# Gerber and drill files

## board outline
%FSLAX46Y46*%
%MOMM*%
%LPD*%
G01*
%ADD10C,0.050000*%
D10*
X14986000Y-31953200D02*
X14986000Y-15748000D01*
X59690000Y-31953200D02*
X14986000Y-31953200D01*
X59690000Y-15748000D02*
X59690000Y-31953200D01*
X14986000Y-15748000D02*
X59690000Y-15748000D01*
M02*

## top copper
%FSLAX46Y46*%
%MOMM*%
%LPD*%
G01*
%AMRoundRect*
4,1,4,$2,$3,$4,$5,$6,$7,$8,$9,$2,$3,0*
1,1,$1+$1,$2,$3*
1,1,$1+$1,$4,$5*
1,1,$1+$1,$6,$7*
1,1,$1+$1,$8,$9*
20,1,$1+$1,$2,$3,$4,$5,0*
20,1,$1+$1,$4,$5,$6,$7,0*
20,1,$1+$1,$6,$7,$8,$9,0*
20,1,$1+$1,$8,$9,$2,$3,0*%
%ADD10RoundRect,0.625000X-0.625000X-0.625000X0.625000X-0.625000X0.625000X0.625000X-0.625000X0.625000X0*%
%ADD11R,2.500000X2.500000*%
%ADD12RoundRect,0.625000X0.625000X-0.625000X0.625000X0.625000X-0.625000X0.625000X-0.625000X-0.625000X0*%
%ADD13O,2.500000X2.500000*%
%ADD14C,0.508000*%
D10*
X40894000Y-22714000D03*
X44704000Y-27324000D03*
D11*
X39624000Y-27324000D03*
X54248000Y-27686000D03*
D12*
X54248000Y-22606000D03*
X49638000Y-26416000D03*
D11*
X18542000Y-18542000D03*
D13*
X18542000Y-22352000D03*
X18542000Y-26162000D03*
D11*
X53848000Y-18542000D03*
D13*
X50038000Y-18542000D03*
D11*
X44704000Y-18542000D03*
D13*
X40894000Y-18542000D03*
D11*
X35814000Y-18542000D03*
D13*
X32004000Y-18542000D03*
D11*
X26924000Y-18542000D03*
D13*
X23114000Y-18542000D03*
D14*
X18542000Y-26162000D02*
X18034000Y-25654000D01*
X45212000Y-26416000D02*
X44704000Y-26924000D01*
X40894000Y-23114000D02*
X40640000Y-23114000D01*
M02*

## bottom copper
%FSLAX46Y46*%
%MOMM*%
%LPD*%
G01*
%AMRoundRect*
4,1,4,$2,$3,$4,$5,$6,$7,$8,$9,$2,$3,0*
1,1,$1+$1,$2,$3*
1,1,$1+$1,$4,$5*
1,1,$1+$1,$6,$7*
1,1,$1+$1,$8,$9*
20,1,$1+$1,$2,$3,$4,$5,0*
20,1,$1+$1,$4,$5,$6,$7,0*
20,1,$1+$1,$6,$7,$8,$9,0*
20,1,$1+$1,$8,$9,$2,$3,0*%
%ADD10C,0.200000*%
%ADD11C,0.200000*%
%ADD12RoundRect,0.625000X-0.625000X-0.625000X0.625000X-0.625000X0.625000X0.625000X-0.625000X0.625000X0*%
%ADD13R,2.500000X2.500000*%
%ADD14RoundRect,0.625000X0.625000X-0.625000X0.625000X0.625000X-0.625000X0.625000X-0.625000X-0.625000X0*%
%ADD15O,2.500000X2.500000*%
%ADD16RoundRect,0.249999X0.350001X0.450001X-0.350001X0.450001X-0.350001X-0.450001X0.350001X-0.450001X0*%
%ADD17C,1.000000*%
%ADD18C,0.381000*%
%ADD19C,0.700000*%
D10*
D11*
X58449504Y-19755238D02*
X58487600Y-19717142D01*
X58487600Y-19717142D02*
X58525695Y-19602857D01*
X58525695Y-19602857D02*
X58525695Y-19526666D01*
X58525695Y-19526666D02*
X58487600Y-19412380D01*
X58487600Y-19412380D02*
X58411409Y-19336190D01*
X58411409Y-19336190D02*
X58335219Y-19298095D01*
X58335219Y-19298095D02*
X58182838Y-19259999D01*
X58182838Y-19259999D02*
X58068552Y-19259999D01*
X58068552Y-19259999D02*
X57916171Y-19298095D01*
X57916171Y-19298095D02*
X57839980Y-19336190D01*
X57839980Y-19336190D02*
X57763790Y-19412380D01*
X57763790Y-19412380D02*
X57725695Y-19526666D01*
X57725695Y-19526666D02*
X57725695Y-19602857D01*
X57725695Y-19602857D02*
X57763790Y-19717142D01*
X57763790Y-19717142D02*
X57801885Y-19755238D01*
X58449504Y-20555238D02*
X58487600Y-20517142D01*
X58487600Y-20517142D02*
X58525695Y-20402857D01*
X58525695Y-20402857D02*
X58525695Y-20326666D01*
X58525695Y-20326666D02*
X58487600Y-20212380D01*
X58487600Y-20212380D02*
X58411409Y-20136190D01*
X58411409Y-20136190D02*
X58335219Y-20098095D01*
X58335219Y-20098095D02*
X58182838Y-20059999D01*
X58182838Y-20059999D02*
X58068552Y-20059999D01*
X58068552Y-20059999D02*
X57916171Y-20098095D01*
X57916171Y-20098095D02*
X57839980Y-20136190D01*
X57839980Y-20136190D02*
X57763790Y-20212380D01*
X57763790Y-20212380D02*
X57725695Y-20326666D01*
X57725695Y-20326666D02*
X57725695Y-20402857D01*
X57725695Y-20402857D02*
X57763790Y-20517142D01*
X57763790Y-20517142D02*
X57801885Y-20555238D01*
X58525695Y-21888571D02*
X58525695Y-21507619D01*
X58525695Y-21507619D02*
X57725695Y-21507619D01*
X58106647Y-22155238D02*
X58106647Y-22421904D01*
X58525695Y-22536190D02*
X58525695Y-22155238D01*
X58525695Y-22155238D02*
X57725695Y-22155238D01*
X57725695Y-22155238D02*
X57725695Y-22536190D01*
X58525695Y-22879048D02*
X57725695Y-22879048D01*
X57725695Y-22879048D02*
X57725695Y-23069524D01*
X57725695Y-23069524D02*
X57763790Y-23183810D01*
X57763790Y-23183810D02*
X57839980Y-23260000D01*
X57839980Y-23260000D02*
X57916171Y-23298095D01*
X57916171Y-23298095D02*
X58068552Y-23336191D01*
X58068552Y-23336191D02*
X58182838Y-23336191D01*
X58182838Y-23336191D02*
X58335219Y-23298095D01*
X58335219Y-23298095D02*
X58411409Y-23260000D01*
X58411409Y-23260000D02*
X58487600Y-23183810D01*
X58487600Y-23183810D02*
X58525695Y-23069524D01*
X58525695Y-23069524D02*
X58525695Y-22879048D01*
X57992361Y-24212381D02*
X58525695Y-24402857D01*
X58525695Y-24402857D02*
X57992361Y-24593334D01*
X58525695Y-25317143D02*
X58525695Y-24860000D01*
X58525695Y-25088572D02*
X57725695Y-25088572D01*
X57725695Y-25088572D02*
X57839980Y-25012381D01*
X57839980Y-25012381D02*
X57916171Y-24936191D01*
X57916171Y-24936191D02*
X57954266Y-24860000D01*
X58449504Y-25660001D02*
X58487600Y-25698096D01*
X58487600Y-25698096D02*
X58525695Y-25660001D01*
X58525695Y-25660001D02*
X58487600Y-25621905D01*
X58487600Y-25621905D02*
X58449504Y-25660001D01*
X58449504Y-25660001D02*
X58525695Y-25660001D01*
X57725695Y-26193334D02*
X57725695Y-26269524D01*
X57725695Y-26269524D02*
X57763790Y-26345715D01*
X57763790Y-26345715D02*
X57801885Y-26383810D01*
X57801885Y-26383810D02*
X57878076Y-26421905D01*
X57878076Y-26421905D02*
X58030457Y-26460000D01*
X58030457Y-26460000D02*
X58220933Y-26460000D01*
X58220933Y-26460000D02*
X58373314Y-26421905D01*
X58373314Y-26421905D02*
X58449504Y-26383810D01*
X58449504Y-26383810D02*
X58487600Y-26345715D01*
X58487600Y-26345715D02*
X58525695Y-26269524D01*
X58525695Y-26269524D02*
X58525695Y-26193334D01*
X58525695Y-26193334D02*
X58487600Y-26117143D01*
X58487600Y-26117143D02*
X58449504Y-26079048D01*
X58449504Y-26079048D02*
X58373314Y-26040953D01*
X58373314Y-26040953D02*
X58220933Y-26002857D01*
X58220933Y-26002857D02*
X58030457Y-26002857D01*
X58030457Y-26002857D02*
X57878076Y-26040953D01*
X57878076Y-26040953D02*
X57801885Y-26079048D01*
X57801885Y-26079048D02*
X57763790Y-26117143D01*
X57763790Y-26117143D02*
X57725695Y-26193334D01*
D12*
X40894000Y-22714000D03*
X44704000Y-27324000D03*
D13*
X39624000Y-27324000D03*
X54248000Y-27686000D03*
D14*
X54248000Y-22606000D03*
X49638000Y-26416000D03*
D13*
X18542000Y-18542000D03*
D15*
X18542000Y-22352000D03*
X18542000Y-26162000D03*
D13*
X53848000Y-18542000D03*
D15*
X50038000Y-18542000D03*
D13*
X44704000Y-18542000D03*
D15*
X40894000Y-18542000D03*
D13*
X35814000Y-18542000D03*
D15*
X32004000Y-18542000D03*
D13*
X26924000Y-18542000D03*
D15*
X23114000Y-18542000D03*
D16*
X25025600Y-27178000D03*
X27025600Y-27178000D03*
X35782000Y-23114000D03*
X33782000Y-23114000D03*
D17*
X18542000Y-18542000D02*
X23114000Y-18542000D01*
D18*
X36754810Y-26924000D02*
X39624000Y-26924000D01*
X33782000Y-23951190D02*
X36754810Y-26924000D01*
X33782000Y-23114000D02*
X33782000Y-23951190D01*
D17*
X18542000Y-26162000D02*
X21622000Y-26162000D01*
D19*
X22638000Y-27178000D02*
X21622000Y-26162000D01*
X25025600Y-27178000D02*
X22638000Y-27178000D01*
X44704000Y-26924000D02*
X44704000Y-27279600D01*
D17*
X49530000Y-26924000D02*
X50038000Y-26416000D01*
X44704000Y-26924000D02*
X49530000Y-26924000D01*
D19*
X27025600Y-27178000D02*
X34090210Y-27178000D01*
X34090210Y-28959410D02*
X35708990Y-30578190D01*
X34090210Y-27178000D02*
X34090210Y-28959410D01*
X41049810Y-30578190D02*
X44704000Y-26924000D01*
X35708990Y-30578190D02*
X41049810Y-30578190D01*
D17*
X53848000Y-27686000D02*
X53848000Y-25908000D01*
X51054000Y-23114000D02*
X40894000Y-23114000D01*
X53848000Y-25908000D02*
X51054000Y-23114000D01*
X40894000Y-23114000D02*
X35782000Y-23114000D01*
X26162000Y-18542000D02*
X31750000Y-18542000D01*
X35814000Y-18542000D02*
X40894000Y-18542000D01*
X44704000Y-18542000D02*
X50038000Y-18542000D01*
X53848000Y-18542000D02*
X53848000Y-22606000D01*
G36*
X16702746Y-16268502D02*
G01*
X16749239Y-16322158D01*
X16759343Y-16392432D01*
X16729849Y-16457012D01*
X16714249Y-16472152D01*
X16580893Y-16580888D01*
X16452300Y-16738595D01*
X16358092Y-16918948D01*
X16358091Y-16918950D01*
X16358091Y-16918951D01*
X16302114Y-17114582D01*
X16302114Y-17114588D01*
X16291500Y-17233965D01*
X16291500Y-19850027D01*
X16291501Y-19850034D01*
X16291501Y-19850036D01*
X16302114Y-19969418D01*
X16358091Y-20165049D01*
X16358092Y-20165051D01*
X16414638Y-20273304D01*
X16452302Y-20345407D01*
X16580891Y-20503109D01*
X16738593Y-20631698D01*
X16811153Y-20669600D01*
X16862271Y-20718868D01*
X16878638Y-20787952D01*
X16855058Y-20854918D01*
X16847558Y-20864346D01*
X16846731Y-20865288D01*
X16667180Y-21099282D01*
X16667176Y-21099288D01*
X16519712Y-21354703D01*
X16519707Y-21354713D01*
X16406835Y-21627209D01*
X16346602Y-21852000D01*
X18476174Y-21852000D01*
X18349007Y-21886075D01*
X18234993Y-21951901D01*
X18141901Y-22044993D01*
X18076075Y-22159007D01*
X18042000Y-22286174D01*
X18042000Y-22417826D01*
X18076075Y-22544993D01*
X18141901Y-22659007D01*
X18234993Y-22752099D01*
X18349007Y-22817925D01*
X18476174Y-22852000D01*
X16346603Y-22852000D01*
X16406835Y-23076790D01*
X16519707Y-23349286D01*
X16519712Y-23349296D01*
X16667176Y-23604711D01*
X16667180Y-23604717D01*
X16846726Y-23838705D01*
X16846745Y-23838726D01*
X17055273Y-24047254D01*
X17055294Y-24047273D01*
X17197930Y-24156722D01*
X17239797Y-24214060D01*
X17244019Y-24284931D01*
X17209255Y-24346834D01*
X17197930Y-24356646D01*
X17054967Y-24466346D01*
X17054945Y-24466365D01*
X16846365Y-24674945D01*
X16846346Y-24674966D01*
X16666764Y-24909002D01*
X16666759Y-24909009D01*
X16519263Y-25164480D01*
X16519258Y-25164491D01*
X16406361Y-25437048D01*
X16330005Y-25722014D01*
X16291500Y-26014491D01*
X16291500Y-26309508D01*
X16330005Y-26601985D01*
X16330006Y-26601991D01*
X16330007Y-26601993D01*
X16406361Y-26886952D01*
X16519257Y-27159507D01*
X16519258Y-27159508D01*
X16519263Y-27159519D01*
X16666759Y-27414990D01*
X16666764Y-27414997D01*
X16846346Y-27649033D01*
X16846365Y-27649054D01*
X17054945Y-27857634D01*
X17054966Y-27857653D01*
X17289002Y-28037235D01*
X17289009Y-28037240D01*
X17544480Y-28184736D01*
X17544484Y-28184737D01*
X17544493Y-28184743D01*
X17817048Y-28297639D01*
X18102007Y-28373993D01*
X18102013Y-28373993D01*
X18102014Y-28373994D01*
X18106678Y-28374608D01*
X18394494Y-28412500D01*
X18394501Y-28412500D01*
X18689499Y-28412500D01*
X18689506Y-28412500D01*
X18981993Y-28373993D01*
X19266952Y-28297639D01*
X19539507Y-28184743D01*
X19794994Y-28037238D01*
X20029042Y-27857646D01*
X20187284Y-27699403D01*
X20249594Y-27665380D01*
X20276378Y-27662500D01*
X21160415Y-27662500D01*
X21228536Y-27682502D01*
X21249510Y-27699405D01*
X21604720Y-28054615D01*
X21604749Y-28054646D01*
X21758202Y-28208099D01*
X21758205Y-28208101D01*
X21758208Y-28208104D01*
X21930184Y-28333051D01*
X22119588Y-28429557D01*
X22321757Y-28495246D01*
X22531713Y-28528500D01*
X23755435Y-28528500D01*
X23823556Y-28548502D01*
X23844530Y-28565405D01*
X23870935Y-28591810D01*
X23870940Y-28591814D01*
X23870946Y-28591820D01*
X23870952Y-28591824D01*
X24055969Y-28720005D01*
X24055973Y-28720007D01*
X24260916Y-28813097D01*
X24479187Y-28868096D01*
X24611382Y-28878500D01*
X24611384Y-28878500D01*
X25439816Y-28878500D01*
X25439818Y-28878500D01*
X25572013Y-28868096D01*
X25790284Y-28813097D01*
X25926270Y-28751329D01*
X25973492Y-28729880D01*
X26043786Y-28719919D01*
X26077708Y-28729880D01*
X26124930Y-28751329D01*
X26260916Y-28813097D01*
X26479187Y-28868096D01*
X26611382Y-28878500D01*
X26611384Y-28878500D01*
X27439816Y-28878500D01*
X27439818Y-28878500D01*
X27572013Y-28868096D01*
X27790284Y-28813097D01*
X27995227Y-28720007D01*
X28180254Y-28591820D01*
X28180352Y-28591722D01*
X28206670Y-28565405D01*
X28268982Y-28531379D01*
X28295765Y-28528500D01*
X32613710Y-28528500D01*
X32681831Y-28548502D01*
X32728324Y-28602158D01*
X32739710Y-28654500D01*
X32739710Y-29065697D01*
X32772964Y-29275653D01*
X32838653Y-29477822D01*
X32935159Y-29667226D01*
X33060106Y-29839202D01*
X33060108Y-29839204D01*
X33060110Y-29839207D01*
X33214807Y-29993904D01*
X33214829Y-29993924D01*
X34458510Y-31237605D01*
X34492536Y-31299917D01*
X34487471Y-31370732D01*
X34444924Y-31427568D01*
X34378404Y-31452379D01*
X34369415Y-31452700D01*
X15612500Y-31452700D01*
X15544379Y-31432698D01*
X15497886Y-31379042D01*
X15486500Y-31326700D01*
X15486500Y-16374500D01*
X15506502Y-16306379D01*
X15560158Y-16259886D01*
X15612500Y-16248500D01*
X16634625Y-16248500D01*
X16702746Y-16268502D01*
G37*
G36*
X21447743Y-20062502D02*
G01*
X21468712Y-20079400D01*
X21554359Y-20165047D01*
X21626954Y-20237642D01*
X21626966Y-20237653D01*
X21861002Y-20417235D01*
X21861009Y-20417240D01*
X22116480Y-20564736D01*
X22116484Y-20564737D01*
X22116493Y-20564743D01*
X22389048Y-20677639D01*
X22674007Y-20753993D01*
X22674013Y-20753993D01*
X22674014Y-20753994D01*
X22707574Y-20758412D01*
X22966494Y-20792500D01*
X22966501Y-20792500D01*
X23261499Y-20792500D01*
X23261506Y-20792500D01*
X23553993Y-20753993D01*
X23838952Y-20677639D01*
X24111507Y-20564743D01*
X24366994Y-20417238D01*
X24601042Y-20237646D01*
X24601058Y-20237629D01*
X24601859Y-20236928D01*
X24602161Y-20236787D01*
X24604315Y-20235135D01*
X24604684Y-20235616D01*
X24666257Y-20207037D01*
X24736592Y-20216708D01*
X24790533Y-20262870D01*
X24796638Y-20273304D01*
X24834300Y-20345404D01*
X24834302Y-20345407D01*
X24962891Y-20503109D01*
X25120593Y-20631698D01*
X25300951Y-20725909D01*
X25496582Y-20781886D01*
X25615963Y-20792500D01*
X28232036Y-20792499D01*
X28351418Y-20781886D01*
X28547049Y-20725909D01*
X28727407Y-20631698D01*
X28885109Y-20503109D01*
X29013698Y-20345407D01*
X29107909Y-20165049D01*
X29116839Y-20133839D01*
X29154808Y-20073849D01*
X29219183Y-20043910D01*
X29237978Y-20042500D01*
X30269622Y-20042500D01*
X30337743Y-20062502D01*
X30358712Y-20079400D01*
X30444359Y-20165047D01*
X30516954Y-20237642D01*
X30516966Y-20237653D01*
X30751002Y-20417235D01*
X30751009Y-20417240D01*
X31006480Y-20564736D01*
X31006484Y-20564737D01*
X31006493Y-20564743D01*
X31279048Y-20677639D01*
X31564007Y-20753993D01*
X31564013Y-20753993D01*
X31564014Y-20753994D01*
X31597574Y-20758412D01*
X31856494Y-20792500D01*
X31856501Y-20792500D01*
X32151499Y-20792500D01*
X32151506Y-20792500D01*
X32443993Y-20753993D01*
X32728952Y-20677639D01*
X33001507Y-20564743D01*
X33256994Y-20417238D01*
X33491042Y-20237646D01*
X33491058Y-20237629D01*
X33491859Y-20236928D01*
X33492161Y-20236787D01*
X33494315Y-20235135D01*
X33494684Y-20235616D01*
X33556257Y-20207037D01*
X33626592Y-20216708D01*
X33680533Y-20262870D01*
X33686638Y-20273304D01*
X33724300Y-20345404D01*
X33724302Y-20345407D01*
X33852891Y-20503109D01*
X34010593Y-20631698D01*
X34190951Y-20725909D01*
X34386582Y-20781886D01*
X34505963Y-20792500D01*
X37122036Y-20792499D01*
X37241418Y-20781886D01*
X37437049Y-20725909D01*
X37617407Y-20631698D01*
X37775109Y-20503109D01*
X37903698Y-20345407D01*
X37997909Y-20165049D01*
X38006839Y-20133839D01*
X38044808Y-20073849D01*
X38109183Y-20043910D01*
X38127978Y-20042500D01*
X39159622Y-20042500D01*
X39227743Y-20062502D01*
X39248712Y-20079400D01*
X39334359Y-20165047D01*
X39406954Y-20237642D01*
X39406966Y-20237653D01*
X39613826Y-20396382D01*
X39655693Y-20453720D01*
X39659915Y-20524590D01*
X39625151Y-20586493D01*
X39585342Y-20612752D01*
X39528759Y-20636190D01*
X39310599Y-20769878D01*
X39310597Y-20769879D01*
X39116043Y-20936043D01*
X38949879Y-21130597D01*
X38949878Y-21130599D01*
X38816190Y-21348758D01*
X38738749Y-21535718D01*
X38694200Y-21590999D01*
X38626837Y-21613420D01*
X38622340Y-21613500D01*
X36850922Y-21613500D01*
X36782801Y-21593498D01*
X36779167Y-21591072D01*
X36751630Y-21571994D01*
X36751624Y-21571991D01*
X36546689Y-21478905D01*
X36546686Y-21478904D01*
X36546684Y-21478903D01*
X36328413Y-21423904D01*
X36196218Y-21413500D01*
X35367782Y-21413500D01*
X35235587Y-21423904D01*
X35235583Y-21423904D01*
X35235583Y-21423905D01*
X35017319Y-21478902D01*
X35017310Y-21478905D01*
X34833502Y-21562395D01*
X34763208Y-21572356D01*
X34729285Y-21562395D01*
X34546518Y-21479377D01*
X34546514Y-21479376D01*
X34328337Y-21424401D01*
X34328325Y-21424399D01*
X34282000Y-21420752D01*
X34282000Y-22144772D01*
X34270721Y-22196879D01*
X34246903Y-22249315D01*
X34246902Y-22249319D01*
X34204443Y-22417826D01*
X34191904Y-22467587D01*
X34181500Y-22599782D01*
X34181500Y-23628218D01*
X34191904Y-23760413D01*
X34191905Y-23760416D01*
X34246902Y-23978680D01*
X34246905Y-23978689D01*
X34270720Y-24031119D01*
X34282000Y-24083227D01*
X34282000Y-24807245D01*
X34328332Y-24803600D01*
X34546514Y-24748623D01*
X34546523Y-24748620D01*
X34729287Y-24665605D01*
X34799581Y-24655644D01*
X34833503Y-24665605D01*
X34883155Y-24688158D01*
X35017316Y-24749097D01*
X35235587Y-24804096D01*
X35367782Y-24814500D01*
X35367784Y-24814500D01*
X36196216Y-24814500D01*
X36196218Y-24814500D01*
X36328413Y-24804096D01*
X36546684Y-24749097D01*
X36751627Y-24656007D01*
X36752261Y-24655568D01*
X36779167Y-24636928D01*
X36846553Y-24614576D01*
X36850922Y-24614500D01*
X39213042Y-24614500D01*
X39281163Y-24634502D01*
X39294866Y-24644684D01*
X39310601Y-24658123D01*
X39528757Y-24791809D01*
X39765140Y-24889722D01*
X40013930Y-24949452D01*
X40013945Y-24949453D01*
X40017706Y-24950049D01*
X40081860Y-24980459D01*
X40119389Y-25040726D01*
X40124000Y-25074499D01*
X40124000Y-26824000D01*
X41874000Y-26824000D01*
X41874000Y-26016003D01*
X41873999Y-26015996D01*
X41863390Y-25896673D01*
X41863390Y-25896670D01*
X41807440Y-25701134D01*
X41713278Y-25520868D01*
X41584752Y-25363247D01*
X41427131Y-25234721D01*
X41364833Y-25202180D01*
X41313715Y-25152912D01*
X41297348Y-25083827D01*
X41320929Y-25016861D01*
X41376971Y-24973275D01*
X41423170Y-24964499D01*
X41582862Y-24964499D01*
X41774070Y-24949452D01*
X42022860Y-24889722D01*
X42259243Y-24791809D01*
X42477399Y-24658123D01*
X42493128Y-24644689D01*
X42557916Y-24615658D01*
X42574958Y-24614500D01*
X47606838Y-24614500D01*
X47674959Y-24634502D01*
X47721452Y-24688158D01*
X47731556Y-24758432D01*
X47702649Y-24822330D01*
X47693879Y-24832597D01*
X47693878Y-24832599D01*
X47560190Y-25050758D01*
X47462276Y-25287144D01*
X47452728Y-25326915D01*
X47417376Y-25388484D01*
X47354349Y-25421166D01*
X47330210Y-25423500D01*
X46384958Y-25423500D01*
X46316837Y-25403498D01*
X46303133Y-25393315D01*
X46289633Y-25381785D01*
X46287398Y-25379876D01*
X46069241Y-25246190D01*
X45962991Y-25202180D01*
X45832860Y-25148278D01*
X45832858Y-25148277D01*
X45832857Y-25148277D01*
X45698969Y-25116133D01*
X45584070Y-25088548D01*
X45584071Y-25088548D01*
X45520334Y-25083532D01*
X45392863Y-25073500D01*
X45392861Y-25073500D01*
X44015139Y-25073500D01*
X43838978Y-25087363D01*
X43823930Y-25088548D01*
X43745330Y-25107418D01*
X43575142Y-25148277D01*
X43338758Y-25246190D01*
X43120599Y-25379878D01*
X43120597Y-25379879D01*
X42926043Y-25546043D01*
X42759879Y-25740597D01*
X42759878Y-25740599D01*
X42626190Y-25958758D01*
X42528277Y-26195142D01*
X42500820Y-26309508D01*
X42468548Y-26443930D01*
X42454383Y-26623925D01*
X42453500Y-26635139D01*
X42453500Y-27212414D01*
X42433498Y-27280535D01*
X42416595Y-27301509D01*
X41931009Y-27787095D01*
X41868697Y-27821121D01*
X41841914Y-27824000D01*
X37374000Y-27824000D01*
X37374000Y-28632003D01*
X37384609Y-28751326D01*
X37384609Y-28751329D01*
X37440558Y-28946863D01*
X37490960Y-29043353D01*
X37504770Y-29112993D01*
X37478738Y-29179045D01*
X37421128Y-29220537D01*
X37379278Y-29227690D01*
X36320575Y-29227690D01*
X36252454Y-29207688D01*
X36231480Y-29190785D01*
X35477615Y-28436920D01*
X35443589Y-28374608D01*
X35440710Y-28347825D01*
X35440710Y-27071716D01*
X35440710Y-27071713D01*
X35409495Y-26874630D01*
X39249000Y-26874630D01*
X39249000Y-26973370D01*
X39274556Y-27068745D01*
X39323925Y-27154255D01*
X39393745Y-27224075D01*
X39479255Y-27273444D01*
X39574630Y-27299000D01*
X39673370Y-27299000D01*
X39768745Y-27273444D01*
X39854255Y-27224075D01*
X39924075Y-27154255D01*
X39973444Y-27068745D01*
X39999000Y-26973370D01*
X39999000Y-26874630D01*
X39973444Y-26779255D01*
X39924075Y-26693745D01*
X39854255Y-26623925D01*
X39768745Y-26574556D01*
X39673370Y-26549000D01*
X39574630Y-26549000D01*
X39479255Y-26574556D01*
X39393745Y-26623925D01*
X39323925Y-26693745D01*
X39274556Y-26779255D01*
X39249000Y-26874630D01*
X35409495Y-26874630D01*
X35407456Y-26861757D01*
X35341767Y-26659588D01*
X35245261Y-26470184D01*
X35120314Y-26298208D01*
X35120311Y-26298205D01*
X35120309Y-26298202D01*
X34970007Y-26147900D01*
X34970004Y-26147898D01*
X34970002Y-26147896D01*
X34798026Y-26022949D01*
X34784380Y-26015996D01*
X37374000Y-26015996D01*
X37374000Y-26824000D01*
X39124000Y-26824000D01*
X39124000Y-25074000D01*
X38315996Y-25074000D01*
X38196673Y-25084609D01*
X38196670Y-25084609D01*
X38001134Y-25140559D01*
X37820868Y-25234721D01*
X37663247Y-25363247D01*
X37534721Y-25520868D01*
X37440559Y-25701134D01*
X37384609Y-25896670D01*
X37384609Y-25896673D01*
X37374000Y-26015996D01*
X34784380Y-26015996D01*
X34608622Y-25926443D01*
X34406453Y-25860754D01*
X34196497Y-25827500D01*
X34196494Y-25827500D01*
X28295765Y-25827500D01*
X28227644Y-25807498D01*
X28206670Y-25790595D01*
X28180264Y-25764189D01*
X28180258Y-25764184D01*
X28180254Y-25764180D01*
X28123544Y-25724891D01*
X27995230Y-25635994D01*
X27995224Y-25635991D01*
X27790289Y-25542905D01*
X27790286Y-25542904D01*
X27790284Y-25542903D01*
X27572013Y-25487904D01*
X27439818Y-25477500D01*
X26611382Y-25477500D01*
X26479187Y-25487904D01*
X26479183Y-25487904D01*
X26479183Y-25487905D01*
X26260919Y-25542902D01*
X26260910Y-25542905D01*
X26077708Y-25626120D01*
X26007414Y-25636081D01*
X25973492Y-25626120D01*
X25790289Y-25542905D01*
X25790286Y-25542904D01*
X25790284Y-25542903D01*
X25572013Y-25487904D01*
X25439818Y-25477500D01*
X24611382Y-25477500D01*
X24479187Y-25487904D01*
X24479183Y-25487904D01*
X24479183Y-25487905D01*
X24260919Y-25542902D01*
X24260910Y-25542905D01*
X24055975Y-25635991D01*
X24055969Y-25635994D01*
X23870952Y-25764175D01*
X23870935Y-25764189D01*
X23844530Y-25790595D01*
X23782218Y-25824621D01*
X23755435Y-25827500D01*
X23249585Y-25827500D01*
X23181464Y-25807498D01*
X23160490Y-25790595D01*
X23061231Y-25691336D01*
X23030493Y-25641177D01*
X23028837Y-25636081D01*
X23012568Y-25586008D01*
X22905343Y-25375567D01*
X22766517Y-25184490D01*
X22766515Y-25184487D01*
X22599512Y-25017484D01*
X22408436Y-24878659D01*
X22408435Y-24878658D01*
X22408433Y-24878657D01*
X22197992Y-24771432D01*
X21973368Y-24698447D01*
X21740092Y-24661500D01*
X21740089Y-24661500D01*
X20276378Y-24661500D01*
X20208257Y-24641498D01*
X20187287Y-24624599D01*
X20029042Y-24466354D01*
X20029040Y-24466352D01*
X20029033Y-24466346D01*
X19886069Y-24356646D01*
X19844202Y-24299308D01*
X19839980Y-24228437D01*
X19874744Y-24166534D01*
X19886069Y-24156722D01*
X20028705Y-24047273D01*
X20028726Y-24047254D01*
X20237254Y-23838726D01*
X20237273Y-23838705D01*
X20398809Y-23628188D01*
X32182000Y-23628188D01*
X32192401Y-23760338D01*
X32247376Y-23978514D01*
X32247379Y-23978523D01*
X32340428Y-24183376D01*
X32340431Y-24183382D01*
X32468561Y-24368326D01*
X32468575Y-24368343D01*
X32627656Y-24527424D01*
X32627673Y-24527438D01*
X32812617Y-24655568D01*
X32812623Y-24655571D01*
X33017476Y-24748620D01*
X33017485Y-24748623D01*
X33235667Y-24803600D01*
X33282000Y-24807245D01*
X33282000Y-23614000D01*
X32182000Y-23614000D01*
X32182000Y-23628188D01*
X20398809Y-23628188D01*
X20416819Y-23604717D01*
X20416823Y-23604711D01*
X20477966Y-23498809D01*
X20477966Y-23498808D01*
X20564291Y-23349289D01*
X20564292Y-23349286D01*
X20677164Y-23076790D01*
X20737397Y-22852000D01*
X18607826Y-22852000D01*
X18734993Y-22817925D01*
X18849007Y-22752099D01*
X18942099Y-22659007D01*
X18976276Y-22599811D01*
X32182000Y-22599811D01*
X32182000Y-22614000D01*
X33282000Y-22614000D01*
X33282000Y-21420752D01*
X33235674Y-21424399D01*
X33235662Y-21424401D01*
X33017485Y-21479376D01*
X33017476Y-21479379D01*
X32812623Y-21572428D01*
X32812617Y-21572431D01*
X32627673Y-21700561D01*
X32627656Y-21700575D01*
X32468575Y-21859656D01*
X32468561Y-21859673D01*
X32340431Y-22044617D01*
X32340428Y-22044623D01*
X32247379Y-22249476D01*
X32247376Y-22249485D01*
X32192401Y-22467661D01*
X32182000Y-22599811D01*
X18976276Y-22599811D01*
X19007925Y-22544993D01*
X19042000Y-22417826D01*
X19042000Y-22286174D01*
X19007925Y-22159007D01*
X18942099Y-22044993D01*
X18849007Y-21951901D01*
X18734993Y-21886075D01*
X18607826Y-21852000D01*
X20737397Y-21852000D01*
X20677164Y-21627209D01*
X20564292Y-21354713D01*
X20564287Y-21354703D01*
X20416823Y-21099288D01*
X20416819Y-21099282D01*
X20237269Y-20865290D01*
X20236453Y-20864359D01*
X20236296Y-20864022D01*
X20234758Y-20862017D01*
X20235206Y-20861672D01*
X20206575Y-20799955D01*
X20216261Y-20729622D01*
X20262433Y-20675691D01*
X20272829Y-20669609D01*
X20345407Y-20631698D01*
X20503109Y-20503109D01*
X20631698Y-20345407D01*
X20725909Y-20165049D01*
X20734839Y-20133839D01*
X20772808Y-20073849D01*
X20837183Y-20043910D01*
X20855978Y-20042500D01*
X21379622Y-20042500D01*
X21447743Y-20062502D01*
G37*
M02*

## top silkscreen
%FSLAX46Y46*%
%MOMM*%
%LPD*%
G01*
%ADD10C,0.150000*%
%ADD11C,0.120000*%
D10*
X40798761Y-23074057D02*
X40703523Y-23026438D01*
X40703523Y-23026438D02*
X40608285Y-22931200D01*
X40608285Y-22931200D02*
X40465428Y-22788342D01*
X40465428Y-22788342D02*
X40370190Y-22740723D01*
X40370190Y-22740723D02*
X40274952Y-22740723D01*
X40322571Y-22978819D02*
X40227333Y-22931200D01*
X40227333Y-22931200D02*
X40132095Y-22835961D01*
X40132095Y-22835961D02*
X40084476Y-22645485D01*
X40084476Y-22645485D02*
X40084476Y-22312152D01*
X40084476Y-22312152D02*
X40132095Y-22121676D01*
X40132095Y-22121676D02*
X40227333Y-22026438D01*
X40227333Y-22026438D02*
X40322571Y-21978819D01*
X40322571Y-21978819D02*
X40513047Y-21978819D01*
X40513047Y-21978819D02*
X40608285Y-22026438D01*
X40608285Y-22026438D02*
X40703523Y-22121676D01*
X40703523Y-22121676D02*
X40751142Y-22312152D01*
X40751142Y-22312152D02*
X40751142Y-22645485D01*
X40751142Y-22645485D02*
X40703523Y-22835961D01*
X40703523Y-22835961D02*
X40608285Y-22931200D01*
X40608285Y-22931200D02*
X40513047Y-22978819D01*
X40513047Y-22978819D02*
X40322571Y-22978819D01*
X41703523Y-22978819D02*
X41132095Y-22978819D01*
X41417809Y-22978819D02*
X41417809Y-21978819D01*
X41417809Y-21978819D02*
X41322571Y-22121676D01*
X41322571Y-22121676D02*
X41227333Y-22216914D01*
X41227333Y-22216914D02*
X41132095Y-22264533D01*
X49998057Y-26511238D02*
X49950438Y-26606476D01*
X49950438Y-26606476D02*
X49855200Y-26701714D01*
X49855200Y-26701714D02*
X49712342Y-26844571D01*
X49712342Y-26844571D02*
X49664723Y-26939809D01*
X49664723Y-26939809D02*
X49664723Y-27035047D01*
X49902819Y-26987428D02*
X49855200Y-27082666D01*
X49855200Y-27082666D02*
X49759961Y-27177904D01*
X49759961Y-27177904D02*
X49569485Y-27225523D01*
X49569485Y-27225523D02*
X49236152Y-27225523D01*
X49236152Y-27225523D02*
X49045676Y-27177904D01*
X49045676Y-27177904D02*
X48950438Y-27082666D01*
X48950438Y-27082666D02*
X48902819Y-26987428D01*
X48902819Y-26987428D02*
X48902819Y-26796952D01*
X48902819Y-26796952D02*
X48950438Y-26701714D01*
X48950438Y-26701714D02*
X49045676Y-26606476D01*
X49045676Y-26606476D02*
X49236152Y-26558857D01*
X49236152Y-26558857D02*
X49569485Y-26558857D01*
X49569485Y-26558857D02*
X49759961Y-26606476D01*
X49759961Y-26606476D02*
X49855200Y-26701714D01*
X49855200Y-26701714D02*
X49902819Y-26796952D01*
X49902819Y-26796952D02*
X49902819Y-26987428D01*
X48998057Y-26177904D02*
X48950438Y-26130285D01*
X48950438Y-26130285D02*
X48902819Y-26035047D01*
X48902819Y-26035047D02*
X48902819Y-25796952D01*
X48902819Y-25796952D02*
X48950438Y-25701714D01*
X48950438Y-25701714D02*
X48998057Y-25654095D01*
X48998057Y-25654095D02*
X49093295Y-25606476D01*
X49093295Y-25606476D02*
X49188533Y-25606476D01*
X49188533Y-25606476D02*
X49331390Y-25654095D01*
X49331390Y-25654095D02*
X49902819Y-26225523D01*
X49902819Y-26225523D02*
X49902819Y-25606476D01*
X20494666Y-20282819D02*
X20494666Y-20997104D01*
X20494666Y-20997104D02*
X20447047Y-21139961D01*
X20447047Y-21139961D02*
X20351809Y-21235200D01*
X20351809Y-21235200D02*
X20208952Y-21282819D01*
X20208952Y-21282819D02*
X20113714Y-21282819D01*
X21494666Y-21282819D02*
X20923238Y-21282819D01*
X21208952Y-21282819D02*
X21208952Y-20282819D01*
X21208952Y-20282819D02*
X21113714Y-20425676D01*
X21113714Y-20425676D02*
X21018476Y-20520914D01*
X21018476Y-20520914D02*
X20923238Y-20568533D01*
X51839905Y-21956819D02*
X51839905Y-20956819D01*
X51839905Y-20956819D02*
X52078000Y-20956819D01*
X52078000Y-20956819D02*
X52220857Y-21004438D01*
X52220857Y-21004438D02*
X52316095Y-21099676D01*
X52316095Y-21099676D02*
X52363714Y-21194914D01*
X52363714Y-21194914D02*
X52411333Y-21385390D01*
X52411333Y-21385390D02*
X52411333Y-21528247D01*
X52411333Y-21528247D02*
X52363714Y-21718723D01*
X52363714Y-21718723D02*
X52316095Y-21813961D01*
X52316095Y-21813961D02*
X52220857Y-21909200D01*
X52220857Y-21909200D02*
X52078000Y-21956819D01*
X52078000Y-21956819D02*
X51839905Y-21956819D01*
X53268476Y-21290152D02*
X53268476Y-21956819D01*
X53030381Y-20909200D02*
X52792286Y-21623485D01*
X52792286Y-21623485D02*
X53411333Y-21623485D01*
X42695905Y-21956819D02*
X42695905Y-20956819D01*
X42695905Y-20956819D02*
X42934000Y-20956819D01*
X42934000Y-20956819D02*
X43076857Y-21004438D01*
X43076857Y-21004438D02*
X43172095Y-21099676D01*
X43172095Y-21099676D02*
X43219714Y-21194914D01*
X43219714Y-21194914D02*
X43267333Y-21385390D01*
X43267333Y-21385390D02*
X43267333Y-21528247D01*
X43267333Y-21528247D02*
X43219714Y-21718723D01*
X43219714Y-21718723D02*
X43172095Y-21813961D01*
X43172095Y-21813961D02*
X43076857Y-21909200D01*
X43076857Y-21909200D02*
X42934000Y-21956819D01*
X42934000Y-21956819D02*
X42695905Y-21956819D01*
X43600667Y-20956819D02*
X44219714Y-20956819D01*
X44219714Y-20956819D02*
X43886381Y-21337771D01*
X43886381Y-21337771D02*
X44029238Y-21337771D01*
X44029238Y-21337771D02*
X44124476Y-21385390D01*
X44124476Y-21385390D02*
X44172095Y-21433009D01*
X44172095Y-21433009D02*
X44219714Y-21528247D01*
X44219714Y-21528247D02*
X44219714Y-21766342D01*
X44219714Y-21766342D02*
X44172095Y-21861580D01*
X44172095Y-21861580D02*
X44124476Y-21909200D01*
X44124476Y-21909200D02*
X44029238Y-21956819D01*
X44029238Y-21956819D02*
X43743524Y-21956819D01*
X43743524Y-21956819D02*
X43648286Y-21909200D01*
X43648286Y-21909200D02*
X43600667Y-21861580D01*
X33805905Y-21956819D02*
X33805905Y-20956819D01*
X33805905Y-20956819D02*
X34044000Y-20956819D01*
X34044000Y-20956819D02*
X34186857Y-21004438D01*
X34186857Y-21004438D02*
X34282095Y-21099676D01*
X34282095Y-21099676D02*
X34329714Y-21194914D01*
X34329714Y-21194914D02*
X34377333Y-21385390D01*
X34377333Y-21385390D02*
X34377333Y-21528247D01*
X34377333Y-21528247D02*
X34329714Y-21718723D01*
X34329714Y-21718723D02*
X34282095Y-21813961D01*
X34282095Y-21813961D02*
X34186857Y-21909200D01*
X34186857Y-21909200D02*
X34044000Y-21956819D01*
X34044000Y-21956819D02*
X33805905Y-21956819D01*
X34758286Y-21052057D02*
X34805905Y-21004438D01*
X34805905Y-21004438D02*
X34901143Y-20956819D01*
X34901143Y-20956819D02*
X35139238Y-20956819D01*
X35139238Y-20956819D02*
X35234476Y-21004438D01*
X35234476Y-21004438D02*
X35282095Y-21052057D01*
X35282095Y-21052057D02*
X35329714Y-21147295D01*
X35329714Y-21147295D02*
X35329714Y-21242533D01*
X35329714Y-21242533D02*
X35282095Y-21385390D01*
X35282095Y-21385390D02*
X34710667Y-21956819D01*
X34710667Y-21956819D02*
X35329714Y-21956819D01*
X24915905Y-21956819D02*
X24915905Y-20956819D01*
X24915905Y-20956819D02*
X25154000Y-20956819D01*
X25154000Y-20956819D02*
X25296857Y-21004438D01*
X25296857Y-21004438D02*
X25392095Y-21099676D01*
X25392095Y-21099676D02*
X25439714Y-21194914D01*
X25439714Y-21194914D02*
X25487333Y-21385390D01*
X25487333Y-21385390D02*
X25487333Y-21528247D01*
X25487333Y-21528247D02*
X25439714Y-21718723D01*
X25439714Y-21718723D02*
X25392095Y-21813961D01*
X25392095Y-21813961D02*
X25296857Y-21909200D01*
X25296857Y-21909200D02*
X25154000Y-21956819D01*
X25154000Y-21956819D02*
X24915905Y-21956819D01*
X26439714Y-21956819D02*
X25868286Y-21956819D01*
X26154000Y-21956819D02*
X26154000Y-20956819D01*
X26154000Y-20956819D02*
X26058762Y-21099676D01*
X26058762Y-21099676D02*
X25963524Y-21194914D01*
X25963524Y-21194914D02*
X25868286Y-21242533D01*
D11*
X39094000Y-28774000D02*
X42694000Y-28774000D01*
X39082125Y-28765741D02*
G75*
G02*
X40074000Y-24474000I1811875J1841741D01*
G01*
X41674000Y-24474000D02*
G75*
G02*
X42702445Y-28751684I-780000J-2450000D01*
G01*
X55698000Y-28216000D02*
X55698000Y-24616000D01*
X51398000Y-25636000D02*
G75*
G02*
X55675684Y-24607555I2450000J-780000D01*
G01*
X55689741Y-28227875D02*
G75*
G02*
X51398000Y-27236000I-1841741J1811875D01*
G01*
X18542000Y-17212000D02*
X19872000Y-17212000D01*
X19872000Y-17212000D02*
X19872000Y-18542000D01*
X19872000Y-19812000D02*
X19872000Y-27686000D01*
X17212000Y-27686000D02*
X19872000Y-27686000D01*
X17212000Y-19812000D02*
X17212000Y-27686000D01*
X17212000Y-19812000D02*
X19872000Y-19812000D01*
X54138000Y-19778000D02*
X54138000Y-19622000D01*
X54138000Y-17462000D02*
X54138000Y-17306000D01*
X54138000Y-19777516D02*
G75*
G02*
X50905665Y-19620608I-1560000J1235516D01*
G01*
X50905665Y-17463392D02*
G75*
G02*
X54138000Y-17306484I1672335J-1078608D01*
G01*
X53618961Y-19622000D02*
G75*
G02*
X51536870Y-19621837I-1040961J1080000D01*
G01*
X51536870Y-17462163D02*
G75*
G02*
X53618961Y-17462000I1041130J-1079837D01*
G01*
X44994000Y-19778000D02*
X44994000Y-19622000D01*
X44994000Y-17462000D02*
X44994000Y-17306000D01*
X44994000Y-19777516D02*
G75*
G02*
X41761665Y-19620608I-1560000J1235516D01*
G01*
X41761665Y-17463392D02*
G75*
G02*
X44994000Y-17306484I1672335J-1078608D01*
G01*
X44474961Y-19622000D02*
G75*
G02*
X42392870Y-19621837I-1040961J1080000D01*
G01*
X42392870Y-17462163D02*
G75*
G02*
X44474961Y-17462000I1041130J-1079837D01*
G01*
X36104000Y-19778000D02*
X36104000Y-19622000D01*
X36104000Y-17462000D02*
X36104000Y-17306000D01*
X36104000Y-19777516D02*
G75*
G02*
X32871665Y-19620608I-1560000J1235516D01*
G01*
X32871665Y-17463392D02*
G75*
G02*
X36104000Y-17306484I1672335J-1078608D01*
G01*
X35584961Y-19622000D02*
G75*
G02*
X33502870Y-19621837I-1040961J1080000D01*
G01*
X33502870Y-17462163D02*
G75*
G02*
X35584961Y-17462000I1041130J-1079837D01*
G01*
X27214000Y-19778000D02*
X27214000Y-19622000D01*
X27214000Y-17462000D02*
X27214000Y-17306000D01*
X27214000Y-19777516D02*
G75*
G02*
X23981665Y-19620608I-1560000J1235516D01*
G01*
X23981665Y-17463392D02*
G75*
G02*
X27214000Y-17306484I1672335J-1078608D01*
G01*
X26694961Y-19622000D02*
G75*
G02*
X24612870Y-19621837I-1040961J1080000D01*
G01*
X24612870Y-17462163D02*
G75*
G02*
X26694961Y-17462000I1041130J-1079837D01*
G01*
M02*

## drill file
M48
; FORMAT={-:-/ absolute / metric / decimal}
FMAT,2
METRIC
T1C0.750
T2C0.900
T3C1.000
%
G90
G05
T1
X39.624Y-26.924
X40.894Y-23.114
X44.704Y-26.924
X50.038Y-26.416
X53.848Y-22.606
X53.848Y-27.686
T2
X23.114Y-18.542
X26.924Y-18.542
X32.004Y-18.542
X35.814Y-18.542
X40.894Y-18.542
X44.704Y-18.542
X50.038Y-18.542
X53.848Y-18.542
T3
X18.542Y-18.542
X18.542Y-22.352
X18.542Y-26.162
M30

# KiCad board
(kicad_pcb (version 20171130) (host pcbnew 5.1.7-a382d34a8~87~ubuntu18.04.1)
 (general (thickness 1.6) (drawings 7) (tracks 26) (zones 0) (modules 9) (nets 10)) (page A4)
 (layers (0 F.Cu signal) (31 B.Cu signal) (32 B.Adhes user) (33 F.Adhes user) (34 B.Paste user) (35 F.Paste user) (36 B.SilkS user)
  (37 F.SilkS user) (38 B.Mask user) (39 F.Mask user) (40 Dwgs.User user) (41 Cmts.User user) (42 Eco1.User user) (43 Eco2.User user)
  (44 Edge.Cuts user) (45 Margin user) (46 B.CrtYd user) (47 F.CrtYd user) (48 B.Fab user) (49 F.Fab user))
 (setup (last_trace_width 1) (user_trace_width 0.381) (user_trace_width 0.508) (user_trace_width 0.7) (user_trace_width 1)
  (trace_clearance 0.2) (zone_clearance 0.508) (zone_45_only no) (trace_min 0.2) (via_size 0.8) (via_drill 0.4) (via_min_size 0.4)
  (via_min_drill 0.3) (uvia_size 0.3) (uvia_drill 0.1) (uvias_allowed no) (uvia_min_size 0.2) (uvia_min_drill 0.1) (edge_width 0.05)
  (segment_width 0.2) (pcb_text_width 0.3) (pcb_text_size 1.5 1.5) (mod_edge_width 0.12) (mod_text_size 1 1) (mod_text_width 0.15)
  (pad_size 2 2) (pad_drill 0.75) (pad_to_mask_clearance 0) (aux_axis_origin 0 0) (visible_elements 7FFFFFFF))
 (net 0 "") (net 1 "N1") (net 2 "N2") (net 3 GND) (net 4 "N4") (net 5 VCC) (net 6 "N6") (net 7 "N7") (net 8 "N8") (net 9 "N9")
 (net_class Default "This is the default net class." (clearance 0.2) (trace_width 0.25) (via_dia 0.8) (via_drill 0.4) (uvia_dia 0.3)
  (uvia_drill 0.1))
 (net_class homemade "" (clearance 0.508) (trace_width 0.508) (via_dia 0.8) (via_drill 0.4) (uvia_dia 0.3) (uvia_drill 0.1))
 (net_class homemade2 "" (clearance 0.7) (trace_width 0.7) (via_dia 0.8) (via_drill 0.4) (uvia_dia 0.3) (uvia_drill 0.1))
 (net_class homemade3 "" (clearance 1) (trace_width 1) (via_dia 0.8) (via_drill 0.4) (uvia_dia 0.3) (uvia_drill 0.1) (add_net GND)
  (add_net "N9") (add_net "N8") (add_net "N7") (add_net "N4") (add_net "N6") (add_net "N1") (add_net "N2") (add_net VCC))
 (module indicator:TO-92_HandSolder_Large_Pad (layer F.Cu) (at 39.624 26.924)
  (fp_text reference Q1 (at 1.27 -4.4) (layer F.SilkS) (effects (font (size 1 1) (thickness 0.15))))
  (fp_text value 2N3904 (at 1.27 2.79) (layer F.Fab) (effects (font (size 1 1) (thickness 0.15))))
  (fp_line (start -0.53 1.85) (end 3.07 1.85) (layer F.SilkS) (width 0.12))
  (fp_arc (start 1.27 0) (end 0.45 -2.45) (angle -116.9632683) (layer F.SilkS) (width 0.12))
  (fp_arc (start 1.27 0) (end 2.05 -2.45) (angle 117.6433766) (layer F.SilkS) (width 0.12))
  (pad 2 thru_hole roundrect (at 1.27 -3.81) (size 2.5 2.5) (drill 0.75 (offset 0 -0.4)) (layers *.Cu *.Mask) (roundrect_rratio 0.25)
   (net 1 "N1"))
  (pad 3 thru_hole roundrect (at 5.08 0) (size 2.5 2.5) (drill 0.75 (offset 0 0.4)) (layers *.Cu *.Mask) (roundrect_rratio 0.25)
   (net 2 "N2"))
  (pad 1 thru_hole rect (at 0 0) (size 2.5 2.5) (drill 0.75 (offset 0 0.4)) (layers *.Cu *.Mask) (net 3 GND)))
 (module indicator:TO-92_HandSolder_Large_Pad (layer F.Cu) (at 53.848 27.686 90)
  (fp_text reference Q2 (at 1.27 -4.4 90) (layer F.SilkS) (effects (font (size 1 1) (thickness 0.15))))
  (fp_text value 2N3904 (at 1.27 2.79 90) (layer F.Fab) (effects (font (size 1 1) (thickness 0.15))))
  (fp_line (start -0.53 1.85) (end 3.07 1.85) (layer F.SilkS) (width 0.12))
  (fp_arc (start 1.27 0) (end 2.05 -2.45) (angle 117.6433766) (layer F.SilkS) (width 0.12))
  (fp_arc (start 1.27 0) (end 0.45 -2.45) (angle -116.9632683) (layer F.SilkS) (width 0.12))
  (pad 1 thru_hole rect (at 0 0 90) (size 2.5 2.5) (drill 0.75 (offset 0 0.4)) (layers *.Cu *.Mask) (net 1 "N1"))
  (pad 3 thru_hole roundrect (at 5.08 0 90) (size 2.5 2.5) (drill 0.75 (offset 0 0.4)) (layers *.Cu *.Mask) (roundrect_rratio 0.25)
   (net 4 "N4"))
  (pad 2 thru_hole roundrect (at 1.27 -3.81 90) (size 2.5 2.5) (drill 0.75 (offset 0 -0.4)) (layers *.Cu *.Mask) (roundrect_rratio 0.25)
   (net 2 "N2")))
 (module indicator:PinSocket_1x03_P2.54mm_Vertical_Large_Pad (layer F.Cu) (at 18.542 18.542)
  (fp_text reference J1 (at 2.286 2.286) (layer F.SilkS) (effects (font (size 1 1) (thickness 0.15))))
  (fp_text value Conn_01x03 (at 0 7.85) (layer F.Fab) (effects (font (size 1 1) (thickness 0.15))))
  (fp_line (start 0 -1.33) (end 1.33 -1.33) (layer F.SilkS) (width 0.12))
  (fp_line (start 1.33 -1.33) (end 1.33 0) (layer F.SilkS) (width 0.12))
  (fp_line (start 1.33 1.27) (end 1.33 9.144) (layer F.SilkS) (width 0.12))
  (fp_line (start -1.33 9.144) (end 1.33 9.144) (layer F.SilkS) (width 0.12))
  (fp_line (start -1.33 1.27) (end -1.33 9.144) (layer F.SilkS) (width 0.12))
  (fp_line (start -1.33 1.27) (end 1.33 1.27) (layer F.SilkS) (width 0.12))
  (pad 1 thru_hole rect (at 0 0) (size 2.5 2.5) (drill 1) (layers *.Cu *.Mask) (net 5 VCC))
  (pad 2 thru_hole oval (at 0 3.81) (size 2.5 2.5) (drill 1) (layers *.Cu *.Mask) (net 3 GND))
  (pad 3 thru_hole oval (at 0 7.62) (size 2.5 2.5) (drill 1) (layers *.Cu *.Mask) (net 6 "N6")))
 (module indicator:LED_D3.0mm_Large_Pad (layer F.Cu) (at 53.848 18.542 180)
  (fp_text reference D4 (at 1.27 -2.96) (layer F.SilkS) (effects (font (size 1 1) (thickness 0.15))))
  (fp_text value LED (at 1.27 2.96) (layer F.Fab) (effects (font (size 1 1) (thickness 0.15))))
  (fp_line (start -0.29 -1.236) (end -0.29 -1.08) (layer F.SilkS) (width 0.12))
  (fp_line (start -0.29 1.08) (end -0.29 1.236) (layer F.SilkS) (width 0.12))
  (fp_arc (start 1.27 0) (end -0.29 -1.235516) (angle 108.8) (layer F.SilkS) (width 0.12))
  (fp_arc (start 1.27 0) (end -0.29 1.235516) (angle -108.8) (layer F.SilkS) (width 0.12))
  (fp_arc (start 1.27 0) (end 0.229039 -1.08) (angle 87.9) (layer F.SilkS) (width 0.12))
  (fp_arc (start 1.27 0) (end 0.229039 1.08) (angle -87.9) (layer F.SilkS) (width 0.12))
  (pad 1 thru_hole rect (at 0 0 180) (size 2.5 2.5) (drill 0.9) (layers *.Cu *.Mask) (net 4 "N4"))
  (pad 2 thru_hole oval (at 3.81 0 180) (size 2.5 2.5) (drill 0.9) (layers *.Cu *.Mask) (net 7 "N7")))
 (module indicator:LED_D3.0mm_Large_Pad (layer F.Cu) (at 44.704 18.542 180)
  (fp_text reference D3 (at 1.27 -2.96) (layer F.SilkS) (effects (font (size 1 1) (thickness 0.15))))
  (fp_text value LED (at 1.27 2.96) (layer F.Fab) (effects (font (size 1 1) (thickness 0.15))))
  (fp_line (start -0.29 -1.236) (end -0.29 -1.08) (layer F.SilkS) (width 0.12))
  (fp_line (start -0.29 1.08) (end -0.29 1.236) (layer F.SilkS) (width 0.12))
  (fp_arc (start 1.27 0) (end -0.29 -1.235516) (angle 108.8) (layer F.SilkS) (width 0.12))
  (fp_arc (start 1.27 0) (end -0.29 1.235516) (angle -108.8) (layer F.SilkS) (width 0.12))
  (fp_arc (start 1.27 0) (end 0.229039 -1.08) (angle 87.9) (layer F.SilkS) (width 0.12))
  (fp_arc (start 1.27 0) (end 0.229039 1.08) (angle -87.9) (layer F.SilkS) (width 0.12))
  (pad 1 thru_hole rect (at 0 0 180) (size 2.5 2.5) (drill 0.9) (layers *.Cu *.Mask) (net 7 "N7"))
  (pad 2 thru_hole oval (at 3.81 0 180) (size 2.5 2.5) (drill 0.9) (layers *.Cu *.Mask) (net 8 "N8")))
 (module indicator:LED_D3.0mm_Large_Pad (layer F.Cu) (at 35.814 18.542 180)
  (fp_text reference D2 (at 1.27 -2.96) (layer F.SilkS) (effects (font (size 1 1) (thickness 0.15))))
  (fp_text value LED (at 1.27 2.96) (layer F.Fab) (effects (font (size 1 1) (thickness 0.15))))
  (fp_line (start -0.29 -1.236) (end -0.29 -1.08) (layer F.SilkS) (width 0.12))
  (fp_line (start -0.29 1.08) (end -0.29 1.236) (layer F.SilkS) (width 0.12))
  (fp_arc (start 1.27 0) (end -0.29 -1.235516) (angle 108.8) (layer F.SilkS) (width 0.12))
  (fp_arc (start 1.27 0) (end -0.29 1.235516) (angle -108.8) (layer F.SilkS) (width 0.12))
  (fp_arc (start 1.27 0) (end 0.229039 -1.08) (angle 87.9) (layer F.SilkS) (width 0.12))
  (fp_arc (start 1.27 0) (end 0.229039 1.08) (angle -87.9) (layer F.SilkS) (width 0.12))
  (pad 1 thru_hole rect (at 0 0 180) (size 2.5 2.5) (drill 0.9) (layers *.Cu *.Mask) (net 8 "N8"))
  (pad 2 thru_hole oval (at 3.81 0 180) (size 2.5 2.5) (drill 0.9) (layers *.Cu *.Mask) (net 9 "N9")))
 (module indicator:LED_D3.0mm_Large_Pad (layer F.Cu) (at 26.924 18.542 180)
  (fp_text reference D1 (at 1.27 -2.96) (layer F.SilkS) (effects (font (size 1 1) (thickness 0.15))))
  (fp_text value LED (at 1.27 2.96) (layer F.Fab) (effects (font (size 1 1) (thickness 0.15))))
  (fp_line (start -0.29 -1.236) (end -0.29 -1.08) (layer F.SilkS) (width 0.12))
  (fp_line (start -0.29 1.08) (end -0.29 1.236) (layer F.SilkS) (width 0.12))
  (fp_arc (start 1.27 0) (end -0.29 -1.235516) (angle 108.8) (layer F.SilkS) (width 0.12))
  (fp_arc (start 1.27 0) (end -0.29 1.235516) (angle -108.8) (layer F.SilkS) (width 0.12))
  (fp_arc (start 1.27 0) (end 0.229039 -1.08) (angle 87.9) (layer F.SilkS) (width 0.12))
  (fp_arc (start 1.27 0) (end 0.229039 1.08) (angle -87.9) (layer F.SilkS) (width 0.12))
  (pad 1 thru_hole rect (at 0 0 180) (size 2.5 2.5) (drill 0.9) (layers *.Cu *.Mask) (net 9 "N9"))
  (pad 2 thru_hole oval (at 3.81 0 180) (size 2.5 2.5) (drill 0.9) (layers *.Cu *.Mask) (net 5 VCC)))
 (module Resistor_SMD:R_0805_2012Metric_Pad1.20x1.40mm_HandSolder (layer B.Cu) (at 26.0256 27.178 180)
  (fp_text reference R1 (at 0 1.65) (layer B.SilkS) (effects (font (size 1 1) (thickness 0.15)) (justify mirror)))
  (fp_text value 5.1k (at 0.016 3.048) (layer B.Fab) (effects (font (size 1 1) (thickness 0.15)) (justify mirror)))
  (pad 2 smd roundrect (at 1 0 180) (size 1.2 1.4) (layers B.Cu B.Paste B.Mask) (roundrect_rratio 0.2083325) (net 6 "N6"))
  (pad 1 smd roundrect (at -1 0 180) (size 1.2 1.4) (layers B.Cu B.Paste B.Mask) (roundrect_rratio 0.2083325) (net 2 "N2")))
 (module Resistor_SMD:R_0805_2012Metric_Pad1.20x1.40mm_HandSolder (layer B.Cu) (at 34.782 23.114 180)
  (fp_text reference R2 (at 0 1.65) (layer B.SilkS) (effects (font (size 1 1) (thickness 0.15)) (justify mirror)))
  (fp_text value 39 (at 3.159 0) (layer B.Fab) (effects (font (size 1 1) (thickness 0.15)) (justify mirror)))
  (pad 1 smd roundrect (at -1 0 180) (size 1.2 1.4) (layers B.Cu B.Paste B.Mask) (roundrect_rratio 0.2083325) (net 1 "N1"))
  (pad 2 smd roundrect (at 1 0 180) (size 1.2 1.4) (layers B.Cu B.Paste B.Mask) (roundrect_rratio 0.2083325) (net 3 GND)))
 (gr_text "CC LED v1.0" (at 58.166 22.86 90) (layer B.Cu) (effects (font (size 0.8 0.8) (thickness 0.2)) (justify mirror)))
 (gr_line (start 14.986 31.9532) (end 14.986 15.748) (layer Edge.Cuts) (width 0.05))
 (gr_line (start 59.69 31.9532) (end 14.986 31.9532) (layer Edge.Cuts) (width 0.05))
 (gr_line (start 59.69 15.748) (end 59.69 31.9532) (layer Edge.Cuts) (width 0.05))
 (gr_line (start 14.986 15.748) (end 59.69 15.748) (layer Edge.Cuts) (width 0.05))
 (segment (start 18.542 18.542) (end 23.114 18.542) (width 1) (layer B.Cu) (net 5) (status 30))
 (segment (start 36.75481 26.924) (end 39.624 26.924) (width 0.381) (layer B.Cu) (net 3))
 (segment (start 33.782 23.95119) (end 36.75481 26.924) (width 0.381) (layer B.Cu) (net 3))
 (segment (start 33.782 23.114) (end 33.782 23.95119) (width 0.381) (layer B.Cu) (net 3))
 (segment (start 18.542 26.162) (end 18.034 25.654) (width 0.508) (layer F.Cu) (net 6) (status 30))
 (segment (start 18.542 26.162) (end 21.622 26.162) (width 1) (layer B.Cu) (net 6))
 (segment (start 22.638 27.178) (end 21.622 26.162) (width 0.7) (layer B.Cu) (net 6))
 (segment (start 25.0256 27.178) (end 22.638 27.178) (width 0.7) (layer B.Cu) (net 6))
 (segment (start 45.212 26.416) (end 44.704 26.924) (width 0.508) (layer F.Cu) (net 2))
 (segment (start 44.704 26.924) (end 44.704 27.2796) (width 0.7) (layer B.Cu) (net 2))
 (segment (start 49.53 26.924) (end 50.038 26.416) (width 1) (layer B.Cu) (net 2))
 (segment (start 44.704 26.924) (end 49.53 26.924) (width 1) (layer B.Cu) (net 2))
 (segment (start 27.0256 27.178) (end 34.09021 27.178) (width 0.7) (layer B.Cu) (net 2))
 (segment (start 34.09021 28.95941) (end 35.70899 30.57819) (width 0.7) (layer B.Cu) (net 2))
 (segment (start 34.09021 27.178) (end 34.09021 28.95941) (width 0.7) (layer B.Cu) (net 2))
 (segment (start 41.04981 30.57819) (end 44.704 26.924) (width 0.7) (layer B.Cu) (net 2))
 (segment (start 35.70899 30.57819) (end 41.04981 30.57819) (width 0.7) (layer B.Cu) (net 2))
 (segment (start 53.848 27.686) (end 53.848 25.908) (width 1) (layer B.Cu) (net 1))
 (segment (start 51.054 23.114) (end 40.894 23.114) (width 1) (layer B.Cu) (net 1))
 (segment (start 53.848 25.908) (end 51.054 23.114) (width 1) (layer B.Cu) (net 1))
 (segment (start 40.894 23.114) (end 40.64 23.114) (width 0.508) (layer F.Cu) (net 1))
 (segment (start 40.894 23.114) (end 35.782 23.114) (width 1) (layer B.Cu) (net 1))
 (segment (start 26.162 18.542) (end 31.75 18.542) (width 1) (layer B.Cu) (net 9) (status 30))
 (segment (start 35.814 18.542) (end 40.894 18.542) (width 1) (layer B.Cu) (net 8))
 (segment (start 44.704 18.542) (end 50.038 18.542) (width 1) (layer B.Cu) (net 7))
 (segment (start 53.848 18.542) (end 53.848 22.606) (width 1) (layer B.Cu) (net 4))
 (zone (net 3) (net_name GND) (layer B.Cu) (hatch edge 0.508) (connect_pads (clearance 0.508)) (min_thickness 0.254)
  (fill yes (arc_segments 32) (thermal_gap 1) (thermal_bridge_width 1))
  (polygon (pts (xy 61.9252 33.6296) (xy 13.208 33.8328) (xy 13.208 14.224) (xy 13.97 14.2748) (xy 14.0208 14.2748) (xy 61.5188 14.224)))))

